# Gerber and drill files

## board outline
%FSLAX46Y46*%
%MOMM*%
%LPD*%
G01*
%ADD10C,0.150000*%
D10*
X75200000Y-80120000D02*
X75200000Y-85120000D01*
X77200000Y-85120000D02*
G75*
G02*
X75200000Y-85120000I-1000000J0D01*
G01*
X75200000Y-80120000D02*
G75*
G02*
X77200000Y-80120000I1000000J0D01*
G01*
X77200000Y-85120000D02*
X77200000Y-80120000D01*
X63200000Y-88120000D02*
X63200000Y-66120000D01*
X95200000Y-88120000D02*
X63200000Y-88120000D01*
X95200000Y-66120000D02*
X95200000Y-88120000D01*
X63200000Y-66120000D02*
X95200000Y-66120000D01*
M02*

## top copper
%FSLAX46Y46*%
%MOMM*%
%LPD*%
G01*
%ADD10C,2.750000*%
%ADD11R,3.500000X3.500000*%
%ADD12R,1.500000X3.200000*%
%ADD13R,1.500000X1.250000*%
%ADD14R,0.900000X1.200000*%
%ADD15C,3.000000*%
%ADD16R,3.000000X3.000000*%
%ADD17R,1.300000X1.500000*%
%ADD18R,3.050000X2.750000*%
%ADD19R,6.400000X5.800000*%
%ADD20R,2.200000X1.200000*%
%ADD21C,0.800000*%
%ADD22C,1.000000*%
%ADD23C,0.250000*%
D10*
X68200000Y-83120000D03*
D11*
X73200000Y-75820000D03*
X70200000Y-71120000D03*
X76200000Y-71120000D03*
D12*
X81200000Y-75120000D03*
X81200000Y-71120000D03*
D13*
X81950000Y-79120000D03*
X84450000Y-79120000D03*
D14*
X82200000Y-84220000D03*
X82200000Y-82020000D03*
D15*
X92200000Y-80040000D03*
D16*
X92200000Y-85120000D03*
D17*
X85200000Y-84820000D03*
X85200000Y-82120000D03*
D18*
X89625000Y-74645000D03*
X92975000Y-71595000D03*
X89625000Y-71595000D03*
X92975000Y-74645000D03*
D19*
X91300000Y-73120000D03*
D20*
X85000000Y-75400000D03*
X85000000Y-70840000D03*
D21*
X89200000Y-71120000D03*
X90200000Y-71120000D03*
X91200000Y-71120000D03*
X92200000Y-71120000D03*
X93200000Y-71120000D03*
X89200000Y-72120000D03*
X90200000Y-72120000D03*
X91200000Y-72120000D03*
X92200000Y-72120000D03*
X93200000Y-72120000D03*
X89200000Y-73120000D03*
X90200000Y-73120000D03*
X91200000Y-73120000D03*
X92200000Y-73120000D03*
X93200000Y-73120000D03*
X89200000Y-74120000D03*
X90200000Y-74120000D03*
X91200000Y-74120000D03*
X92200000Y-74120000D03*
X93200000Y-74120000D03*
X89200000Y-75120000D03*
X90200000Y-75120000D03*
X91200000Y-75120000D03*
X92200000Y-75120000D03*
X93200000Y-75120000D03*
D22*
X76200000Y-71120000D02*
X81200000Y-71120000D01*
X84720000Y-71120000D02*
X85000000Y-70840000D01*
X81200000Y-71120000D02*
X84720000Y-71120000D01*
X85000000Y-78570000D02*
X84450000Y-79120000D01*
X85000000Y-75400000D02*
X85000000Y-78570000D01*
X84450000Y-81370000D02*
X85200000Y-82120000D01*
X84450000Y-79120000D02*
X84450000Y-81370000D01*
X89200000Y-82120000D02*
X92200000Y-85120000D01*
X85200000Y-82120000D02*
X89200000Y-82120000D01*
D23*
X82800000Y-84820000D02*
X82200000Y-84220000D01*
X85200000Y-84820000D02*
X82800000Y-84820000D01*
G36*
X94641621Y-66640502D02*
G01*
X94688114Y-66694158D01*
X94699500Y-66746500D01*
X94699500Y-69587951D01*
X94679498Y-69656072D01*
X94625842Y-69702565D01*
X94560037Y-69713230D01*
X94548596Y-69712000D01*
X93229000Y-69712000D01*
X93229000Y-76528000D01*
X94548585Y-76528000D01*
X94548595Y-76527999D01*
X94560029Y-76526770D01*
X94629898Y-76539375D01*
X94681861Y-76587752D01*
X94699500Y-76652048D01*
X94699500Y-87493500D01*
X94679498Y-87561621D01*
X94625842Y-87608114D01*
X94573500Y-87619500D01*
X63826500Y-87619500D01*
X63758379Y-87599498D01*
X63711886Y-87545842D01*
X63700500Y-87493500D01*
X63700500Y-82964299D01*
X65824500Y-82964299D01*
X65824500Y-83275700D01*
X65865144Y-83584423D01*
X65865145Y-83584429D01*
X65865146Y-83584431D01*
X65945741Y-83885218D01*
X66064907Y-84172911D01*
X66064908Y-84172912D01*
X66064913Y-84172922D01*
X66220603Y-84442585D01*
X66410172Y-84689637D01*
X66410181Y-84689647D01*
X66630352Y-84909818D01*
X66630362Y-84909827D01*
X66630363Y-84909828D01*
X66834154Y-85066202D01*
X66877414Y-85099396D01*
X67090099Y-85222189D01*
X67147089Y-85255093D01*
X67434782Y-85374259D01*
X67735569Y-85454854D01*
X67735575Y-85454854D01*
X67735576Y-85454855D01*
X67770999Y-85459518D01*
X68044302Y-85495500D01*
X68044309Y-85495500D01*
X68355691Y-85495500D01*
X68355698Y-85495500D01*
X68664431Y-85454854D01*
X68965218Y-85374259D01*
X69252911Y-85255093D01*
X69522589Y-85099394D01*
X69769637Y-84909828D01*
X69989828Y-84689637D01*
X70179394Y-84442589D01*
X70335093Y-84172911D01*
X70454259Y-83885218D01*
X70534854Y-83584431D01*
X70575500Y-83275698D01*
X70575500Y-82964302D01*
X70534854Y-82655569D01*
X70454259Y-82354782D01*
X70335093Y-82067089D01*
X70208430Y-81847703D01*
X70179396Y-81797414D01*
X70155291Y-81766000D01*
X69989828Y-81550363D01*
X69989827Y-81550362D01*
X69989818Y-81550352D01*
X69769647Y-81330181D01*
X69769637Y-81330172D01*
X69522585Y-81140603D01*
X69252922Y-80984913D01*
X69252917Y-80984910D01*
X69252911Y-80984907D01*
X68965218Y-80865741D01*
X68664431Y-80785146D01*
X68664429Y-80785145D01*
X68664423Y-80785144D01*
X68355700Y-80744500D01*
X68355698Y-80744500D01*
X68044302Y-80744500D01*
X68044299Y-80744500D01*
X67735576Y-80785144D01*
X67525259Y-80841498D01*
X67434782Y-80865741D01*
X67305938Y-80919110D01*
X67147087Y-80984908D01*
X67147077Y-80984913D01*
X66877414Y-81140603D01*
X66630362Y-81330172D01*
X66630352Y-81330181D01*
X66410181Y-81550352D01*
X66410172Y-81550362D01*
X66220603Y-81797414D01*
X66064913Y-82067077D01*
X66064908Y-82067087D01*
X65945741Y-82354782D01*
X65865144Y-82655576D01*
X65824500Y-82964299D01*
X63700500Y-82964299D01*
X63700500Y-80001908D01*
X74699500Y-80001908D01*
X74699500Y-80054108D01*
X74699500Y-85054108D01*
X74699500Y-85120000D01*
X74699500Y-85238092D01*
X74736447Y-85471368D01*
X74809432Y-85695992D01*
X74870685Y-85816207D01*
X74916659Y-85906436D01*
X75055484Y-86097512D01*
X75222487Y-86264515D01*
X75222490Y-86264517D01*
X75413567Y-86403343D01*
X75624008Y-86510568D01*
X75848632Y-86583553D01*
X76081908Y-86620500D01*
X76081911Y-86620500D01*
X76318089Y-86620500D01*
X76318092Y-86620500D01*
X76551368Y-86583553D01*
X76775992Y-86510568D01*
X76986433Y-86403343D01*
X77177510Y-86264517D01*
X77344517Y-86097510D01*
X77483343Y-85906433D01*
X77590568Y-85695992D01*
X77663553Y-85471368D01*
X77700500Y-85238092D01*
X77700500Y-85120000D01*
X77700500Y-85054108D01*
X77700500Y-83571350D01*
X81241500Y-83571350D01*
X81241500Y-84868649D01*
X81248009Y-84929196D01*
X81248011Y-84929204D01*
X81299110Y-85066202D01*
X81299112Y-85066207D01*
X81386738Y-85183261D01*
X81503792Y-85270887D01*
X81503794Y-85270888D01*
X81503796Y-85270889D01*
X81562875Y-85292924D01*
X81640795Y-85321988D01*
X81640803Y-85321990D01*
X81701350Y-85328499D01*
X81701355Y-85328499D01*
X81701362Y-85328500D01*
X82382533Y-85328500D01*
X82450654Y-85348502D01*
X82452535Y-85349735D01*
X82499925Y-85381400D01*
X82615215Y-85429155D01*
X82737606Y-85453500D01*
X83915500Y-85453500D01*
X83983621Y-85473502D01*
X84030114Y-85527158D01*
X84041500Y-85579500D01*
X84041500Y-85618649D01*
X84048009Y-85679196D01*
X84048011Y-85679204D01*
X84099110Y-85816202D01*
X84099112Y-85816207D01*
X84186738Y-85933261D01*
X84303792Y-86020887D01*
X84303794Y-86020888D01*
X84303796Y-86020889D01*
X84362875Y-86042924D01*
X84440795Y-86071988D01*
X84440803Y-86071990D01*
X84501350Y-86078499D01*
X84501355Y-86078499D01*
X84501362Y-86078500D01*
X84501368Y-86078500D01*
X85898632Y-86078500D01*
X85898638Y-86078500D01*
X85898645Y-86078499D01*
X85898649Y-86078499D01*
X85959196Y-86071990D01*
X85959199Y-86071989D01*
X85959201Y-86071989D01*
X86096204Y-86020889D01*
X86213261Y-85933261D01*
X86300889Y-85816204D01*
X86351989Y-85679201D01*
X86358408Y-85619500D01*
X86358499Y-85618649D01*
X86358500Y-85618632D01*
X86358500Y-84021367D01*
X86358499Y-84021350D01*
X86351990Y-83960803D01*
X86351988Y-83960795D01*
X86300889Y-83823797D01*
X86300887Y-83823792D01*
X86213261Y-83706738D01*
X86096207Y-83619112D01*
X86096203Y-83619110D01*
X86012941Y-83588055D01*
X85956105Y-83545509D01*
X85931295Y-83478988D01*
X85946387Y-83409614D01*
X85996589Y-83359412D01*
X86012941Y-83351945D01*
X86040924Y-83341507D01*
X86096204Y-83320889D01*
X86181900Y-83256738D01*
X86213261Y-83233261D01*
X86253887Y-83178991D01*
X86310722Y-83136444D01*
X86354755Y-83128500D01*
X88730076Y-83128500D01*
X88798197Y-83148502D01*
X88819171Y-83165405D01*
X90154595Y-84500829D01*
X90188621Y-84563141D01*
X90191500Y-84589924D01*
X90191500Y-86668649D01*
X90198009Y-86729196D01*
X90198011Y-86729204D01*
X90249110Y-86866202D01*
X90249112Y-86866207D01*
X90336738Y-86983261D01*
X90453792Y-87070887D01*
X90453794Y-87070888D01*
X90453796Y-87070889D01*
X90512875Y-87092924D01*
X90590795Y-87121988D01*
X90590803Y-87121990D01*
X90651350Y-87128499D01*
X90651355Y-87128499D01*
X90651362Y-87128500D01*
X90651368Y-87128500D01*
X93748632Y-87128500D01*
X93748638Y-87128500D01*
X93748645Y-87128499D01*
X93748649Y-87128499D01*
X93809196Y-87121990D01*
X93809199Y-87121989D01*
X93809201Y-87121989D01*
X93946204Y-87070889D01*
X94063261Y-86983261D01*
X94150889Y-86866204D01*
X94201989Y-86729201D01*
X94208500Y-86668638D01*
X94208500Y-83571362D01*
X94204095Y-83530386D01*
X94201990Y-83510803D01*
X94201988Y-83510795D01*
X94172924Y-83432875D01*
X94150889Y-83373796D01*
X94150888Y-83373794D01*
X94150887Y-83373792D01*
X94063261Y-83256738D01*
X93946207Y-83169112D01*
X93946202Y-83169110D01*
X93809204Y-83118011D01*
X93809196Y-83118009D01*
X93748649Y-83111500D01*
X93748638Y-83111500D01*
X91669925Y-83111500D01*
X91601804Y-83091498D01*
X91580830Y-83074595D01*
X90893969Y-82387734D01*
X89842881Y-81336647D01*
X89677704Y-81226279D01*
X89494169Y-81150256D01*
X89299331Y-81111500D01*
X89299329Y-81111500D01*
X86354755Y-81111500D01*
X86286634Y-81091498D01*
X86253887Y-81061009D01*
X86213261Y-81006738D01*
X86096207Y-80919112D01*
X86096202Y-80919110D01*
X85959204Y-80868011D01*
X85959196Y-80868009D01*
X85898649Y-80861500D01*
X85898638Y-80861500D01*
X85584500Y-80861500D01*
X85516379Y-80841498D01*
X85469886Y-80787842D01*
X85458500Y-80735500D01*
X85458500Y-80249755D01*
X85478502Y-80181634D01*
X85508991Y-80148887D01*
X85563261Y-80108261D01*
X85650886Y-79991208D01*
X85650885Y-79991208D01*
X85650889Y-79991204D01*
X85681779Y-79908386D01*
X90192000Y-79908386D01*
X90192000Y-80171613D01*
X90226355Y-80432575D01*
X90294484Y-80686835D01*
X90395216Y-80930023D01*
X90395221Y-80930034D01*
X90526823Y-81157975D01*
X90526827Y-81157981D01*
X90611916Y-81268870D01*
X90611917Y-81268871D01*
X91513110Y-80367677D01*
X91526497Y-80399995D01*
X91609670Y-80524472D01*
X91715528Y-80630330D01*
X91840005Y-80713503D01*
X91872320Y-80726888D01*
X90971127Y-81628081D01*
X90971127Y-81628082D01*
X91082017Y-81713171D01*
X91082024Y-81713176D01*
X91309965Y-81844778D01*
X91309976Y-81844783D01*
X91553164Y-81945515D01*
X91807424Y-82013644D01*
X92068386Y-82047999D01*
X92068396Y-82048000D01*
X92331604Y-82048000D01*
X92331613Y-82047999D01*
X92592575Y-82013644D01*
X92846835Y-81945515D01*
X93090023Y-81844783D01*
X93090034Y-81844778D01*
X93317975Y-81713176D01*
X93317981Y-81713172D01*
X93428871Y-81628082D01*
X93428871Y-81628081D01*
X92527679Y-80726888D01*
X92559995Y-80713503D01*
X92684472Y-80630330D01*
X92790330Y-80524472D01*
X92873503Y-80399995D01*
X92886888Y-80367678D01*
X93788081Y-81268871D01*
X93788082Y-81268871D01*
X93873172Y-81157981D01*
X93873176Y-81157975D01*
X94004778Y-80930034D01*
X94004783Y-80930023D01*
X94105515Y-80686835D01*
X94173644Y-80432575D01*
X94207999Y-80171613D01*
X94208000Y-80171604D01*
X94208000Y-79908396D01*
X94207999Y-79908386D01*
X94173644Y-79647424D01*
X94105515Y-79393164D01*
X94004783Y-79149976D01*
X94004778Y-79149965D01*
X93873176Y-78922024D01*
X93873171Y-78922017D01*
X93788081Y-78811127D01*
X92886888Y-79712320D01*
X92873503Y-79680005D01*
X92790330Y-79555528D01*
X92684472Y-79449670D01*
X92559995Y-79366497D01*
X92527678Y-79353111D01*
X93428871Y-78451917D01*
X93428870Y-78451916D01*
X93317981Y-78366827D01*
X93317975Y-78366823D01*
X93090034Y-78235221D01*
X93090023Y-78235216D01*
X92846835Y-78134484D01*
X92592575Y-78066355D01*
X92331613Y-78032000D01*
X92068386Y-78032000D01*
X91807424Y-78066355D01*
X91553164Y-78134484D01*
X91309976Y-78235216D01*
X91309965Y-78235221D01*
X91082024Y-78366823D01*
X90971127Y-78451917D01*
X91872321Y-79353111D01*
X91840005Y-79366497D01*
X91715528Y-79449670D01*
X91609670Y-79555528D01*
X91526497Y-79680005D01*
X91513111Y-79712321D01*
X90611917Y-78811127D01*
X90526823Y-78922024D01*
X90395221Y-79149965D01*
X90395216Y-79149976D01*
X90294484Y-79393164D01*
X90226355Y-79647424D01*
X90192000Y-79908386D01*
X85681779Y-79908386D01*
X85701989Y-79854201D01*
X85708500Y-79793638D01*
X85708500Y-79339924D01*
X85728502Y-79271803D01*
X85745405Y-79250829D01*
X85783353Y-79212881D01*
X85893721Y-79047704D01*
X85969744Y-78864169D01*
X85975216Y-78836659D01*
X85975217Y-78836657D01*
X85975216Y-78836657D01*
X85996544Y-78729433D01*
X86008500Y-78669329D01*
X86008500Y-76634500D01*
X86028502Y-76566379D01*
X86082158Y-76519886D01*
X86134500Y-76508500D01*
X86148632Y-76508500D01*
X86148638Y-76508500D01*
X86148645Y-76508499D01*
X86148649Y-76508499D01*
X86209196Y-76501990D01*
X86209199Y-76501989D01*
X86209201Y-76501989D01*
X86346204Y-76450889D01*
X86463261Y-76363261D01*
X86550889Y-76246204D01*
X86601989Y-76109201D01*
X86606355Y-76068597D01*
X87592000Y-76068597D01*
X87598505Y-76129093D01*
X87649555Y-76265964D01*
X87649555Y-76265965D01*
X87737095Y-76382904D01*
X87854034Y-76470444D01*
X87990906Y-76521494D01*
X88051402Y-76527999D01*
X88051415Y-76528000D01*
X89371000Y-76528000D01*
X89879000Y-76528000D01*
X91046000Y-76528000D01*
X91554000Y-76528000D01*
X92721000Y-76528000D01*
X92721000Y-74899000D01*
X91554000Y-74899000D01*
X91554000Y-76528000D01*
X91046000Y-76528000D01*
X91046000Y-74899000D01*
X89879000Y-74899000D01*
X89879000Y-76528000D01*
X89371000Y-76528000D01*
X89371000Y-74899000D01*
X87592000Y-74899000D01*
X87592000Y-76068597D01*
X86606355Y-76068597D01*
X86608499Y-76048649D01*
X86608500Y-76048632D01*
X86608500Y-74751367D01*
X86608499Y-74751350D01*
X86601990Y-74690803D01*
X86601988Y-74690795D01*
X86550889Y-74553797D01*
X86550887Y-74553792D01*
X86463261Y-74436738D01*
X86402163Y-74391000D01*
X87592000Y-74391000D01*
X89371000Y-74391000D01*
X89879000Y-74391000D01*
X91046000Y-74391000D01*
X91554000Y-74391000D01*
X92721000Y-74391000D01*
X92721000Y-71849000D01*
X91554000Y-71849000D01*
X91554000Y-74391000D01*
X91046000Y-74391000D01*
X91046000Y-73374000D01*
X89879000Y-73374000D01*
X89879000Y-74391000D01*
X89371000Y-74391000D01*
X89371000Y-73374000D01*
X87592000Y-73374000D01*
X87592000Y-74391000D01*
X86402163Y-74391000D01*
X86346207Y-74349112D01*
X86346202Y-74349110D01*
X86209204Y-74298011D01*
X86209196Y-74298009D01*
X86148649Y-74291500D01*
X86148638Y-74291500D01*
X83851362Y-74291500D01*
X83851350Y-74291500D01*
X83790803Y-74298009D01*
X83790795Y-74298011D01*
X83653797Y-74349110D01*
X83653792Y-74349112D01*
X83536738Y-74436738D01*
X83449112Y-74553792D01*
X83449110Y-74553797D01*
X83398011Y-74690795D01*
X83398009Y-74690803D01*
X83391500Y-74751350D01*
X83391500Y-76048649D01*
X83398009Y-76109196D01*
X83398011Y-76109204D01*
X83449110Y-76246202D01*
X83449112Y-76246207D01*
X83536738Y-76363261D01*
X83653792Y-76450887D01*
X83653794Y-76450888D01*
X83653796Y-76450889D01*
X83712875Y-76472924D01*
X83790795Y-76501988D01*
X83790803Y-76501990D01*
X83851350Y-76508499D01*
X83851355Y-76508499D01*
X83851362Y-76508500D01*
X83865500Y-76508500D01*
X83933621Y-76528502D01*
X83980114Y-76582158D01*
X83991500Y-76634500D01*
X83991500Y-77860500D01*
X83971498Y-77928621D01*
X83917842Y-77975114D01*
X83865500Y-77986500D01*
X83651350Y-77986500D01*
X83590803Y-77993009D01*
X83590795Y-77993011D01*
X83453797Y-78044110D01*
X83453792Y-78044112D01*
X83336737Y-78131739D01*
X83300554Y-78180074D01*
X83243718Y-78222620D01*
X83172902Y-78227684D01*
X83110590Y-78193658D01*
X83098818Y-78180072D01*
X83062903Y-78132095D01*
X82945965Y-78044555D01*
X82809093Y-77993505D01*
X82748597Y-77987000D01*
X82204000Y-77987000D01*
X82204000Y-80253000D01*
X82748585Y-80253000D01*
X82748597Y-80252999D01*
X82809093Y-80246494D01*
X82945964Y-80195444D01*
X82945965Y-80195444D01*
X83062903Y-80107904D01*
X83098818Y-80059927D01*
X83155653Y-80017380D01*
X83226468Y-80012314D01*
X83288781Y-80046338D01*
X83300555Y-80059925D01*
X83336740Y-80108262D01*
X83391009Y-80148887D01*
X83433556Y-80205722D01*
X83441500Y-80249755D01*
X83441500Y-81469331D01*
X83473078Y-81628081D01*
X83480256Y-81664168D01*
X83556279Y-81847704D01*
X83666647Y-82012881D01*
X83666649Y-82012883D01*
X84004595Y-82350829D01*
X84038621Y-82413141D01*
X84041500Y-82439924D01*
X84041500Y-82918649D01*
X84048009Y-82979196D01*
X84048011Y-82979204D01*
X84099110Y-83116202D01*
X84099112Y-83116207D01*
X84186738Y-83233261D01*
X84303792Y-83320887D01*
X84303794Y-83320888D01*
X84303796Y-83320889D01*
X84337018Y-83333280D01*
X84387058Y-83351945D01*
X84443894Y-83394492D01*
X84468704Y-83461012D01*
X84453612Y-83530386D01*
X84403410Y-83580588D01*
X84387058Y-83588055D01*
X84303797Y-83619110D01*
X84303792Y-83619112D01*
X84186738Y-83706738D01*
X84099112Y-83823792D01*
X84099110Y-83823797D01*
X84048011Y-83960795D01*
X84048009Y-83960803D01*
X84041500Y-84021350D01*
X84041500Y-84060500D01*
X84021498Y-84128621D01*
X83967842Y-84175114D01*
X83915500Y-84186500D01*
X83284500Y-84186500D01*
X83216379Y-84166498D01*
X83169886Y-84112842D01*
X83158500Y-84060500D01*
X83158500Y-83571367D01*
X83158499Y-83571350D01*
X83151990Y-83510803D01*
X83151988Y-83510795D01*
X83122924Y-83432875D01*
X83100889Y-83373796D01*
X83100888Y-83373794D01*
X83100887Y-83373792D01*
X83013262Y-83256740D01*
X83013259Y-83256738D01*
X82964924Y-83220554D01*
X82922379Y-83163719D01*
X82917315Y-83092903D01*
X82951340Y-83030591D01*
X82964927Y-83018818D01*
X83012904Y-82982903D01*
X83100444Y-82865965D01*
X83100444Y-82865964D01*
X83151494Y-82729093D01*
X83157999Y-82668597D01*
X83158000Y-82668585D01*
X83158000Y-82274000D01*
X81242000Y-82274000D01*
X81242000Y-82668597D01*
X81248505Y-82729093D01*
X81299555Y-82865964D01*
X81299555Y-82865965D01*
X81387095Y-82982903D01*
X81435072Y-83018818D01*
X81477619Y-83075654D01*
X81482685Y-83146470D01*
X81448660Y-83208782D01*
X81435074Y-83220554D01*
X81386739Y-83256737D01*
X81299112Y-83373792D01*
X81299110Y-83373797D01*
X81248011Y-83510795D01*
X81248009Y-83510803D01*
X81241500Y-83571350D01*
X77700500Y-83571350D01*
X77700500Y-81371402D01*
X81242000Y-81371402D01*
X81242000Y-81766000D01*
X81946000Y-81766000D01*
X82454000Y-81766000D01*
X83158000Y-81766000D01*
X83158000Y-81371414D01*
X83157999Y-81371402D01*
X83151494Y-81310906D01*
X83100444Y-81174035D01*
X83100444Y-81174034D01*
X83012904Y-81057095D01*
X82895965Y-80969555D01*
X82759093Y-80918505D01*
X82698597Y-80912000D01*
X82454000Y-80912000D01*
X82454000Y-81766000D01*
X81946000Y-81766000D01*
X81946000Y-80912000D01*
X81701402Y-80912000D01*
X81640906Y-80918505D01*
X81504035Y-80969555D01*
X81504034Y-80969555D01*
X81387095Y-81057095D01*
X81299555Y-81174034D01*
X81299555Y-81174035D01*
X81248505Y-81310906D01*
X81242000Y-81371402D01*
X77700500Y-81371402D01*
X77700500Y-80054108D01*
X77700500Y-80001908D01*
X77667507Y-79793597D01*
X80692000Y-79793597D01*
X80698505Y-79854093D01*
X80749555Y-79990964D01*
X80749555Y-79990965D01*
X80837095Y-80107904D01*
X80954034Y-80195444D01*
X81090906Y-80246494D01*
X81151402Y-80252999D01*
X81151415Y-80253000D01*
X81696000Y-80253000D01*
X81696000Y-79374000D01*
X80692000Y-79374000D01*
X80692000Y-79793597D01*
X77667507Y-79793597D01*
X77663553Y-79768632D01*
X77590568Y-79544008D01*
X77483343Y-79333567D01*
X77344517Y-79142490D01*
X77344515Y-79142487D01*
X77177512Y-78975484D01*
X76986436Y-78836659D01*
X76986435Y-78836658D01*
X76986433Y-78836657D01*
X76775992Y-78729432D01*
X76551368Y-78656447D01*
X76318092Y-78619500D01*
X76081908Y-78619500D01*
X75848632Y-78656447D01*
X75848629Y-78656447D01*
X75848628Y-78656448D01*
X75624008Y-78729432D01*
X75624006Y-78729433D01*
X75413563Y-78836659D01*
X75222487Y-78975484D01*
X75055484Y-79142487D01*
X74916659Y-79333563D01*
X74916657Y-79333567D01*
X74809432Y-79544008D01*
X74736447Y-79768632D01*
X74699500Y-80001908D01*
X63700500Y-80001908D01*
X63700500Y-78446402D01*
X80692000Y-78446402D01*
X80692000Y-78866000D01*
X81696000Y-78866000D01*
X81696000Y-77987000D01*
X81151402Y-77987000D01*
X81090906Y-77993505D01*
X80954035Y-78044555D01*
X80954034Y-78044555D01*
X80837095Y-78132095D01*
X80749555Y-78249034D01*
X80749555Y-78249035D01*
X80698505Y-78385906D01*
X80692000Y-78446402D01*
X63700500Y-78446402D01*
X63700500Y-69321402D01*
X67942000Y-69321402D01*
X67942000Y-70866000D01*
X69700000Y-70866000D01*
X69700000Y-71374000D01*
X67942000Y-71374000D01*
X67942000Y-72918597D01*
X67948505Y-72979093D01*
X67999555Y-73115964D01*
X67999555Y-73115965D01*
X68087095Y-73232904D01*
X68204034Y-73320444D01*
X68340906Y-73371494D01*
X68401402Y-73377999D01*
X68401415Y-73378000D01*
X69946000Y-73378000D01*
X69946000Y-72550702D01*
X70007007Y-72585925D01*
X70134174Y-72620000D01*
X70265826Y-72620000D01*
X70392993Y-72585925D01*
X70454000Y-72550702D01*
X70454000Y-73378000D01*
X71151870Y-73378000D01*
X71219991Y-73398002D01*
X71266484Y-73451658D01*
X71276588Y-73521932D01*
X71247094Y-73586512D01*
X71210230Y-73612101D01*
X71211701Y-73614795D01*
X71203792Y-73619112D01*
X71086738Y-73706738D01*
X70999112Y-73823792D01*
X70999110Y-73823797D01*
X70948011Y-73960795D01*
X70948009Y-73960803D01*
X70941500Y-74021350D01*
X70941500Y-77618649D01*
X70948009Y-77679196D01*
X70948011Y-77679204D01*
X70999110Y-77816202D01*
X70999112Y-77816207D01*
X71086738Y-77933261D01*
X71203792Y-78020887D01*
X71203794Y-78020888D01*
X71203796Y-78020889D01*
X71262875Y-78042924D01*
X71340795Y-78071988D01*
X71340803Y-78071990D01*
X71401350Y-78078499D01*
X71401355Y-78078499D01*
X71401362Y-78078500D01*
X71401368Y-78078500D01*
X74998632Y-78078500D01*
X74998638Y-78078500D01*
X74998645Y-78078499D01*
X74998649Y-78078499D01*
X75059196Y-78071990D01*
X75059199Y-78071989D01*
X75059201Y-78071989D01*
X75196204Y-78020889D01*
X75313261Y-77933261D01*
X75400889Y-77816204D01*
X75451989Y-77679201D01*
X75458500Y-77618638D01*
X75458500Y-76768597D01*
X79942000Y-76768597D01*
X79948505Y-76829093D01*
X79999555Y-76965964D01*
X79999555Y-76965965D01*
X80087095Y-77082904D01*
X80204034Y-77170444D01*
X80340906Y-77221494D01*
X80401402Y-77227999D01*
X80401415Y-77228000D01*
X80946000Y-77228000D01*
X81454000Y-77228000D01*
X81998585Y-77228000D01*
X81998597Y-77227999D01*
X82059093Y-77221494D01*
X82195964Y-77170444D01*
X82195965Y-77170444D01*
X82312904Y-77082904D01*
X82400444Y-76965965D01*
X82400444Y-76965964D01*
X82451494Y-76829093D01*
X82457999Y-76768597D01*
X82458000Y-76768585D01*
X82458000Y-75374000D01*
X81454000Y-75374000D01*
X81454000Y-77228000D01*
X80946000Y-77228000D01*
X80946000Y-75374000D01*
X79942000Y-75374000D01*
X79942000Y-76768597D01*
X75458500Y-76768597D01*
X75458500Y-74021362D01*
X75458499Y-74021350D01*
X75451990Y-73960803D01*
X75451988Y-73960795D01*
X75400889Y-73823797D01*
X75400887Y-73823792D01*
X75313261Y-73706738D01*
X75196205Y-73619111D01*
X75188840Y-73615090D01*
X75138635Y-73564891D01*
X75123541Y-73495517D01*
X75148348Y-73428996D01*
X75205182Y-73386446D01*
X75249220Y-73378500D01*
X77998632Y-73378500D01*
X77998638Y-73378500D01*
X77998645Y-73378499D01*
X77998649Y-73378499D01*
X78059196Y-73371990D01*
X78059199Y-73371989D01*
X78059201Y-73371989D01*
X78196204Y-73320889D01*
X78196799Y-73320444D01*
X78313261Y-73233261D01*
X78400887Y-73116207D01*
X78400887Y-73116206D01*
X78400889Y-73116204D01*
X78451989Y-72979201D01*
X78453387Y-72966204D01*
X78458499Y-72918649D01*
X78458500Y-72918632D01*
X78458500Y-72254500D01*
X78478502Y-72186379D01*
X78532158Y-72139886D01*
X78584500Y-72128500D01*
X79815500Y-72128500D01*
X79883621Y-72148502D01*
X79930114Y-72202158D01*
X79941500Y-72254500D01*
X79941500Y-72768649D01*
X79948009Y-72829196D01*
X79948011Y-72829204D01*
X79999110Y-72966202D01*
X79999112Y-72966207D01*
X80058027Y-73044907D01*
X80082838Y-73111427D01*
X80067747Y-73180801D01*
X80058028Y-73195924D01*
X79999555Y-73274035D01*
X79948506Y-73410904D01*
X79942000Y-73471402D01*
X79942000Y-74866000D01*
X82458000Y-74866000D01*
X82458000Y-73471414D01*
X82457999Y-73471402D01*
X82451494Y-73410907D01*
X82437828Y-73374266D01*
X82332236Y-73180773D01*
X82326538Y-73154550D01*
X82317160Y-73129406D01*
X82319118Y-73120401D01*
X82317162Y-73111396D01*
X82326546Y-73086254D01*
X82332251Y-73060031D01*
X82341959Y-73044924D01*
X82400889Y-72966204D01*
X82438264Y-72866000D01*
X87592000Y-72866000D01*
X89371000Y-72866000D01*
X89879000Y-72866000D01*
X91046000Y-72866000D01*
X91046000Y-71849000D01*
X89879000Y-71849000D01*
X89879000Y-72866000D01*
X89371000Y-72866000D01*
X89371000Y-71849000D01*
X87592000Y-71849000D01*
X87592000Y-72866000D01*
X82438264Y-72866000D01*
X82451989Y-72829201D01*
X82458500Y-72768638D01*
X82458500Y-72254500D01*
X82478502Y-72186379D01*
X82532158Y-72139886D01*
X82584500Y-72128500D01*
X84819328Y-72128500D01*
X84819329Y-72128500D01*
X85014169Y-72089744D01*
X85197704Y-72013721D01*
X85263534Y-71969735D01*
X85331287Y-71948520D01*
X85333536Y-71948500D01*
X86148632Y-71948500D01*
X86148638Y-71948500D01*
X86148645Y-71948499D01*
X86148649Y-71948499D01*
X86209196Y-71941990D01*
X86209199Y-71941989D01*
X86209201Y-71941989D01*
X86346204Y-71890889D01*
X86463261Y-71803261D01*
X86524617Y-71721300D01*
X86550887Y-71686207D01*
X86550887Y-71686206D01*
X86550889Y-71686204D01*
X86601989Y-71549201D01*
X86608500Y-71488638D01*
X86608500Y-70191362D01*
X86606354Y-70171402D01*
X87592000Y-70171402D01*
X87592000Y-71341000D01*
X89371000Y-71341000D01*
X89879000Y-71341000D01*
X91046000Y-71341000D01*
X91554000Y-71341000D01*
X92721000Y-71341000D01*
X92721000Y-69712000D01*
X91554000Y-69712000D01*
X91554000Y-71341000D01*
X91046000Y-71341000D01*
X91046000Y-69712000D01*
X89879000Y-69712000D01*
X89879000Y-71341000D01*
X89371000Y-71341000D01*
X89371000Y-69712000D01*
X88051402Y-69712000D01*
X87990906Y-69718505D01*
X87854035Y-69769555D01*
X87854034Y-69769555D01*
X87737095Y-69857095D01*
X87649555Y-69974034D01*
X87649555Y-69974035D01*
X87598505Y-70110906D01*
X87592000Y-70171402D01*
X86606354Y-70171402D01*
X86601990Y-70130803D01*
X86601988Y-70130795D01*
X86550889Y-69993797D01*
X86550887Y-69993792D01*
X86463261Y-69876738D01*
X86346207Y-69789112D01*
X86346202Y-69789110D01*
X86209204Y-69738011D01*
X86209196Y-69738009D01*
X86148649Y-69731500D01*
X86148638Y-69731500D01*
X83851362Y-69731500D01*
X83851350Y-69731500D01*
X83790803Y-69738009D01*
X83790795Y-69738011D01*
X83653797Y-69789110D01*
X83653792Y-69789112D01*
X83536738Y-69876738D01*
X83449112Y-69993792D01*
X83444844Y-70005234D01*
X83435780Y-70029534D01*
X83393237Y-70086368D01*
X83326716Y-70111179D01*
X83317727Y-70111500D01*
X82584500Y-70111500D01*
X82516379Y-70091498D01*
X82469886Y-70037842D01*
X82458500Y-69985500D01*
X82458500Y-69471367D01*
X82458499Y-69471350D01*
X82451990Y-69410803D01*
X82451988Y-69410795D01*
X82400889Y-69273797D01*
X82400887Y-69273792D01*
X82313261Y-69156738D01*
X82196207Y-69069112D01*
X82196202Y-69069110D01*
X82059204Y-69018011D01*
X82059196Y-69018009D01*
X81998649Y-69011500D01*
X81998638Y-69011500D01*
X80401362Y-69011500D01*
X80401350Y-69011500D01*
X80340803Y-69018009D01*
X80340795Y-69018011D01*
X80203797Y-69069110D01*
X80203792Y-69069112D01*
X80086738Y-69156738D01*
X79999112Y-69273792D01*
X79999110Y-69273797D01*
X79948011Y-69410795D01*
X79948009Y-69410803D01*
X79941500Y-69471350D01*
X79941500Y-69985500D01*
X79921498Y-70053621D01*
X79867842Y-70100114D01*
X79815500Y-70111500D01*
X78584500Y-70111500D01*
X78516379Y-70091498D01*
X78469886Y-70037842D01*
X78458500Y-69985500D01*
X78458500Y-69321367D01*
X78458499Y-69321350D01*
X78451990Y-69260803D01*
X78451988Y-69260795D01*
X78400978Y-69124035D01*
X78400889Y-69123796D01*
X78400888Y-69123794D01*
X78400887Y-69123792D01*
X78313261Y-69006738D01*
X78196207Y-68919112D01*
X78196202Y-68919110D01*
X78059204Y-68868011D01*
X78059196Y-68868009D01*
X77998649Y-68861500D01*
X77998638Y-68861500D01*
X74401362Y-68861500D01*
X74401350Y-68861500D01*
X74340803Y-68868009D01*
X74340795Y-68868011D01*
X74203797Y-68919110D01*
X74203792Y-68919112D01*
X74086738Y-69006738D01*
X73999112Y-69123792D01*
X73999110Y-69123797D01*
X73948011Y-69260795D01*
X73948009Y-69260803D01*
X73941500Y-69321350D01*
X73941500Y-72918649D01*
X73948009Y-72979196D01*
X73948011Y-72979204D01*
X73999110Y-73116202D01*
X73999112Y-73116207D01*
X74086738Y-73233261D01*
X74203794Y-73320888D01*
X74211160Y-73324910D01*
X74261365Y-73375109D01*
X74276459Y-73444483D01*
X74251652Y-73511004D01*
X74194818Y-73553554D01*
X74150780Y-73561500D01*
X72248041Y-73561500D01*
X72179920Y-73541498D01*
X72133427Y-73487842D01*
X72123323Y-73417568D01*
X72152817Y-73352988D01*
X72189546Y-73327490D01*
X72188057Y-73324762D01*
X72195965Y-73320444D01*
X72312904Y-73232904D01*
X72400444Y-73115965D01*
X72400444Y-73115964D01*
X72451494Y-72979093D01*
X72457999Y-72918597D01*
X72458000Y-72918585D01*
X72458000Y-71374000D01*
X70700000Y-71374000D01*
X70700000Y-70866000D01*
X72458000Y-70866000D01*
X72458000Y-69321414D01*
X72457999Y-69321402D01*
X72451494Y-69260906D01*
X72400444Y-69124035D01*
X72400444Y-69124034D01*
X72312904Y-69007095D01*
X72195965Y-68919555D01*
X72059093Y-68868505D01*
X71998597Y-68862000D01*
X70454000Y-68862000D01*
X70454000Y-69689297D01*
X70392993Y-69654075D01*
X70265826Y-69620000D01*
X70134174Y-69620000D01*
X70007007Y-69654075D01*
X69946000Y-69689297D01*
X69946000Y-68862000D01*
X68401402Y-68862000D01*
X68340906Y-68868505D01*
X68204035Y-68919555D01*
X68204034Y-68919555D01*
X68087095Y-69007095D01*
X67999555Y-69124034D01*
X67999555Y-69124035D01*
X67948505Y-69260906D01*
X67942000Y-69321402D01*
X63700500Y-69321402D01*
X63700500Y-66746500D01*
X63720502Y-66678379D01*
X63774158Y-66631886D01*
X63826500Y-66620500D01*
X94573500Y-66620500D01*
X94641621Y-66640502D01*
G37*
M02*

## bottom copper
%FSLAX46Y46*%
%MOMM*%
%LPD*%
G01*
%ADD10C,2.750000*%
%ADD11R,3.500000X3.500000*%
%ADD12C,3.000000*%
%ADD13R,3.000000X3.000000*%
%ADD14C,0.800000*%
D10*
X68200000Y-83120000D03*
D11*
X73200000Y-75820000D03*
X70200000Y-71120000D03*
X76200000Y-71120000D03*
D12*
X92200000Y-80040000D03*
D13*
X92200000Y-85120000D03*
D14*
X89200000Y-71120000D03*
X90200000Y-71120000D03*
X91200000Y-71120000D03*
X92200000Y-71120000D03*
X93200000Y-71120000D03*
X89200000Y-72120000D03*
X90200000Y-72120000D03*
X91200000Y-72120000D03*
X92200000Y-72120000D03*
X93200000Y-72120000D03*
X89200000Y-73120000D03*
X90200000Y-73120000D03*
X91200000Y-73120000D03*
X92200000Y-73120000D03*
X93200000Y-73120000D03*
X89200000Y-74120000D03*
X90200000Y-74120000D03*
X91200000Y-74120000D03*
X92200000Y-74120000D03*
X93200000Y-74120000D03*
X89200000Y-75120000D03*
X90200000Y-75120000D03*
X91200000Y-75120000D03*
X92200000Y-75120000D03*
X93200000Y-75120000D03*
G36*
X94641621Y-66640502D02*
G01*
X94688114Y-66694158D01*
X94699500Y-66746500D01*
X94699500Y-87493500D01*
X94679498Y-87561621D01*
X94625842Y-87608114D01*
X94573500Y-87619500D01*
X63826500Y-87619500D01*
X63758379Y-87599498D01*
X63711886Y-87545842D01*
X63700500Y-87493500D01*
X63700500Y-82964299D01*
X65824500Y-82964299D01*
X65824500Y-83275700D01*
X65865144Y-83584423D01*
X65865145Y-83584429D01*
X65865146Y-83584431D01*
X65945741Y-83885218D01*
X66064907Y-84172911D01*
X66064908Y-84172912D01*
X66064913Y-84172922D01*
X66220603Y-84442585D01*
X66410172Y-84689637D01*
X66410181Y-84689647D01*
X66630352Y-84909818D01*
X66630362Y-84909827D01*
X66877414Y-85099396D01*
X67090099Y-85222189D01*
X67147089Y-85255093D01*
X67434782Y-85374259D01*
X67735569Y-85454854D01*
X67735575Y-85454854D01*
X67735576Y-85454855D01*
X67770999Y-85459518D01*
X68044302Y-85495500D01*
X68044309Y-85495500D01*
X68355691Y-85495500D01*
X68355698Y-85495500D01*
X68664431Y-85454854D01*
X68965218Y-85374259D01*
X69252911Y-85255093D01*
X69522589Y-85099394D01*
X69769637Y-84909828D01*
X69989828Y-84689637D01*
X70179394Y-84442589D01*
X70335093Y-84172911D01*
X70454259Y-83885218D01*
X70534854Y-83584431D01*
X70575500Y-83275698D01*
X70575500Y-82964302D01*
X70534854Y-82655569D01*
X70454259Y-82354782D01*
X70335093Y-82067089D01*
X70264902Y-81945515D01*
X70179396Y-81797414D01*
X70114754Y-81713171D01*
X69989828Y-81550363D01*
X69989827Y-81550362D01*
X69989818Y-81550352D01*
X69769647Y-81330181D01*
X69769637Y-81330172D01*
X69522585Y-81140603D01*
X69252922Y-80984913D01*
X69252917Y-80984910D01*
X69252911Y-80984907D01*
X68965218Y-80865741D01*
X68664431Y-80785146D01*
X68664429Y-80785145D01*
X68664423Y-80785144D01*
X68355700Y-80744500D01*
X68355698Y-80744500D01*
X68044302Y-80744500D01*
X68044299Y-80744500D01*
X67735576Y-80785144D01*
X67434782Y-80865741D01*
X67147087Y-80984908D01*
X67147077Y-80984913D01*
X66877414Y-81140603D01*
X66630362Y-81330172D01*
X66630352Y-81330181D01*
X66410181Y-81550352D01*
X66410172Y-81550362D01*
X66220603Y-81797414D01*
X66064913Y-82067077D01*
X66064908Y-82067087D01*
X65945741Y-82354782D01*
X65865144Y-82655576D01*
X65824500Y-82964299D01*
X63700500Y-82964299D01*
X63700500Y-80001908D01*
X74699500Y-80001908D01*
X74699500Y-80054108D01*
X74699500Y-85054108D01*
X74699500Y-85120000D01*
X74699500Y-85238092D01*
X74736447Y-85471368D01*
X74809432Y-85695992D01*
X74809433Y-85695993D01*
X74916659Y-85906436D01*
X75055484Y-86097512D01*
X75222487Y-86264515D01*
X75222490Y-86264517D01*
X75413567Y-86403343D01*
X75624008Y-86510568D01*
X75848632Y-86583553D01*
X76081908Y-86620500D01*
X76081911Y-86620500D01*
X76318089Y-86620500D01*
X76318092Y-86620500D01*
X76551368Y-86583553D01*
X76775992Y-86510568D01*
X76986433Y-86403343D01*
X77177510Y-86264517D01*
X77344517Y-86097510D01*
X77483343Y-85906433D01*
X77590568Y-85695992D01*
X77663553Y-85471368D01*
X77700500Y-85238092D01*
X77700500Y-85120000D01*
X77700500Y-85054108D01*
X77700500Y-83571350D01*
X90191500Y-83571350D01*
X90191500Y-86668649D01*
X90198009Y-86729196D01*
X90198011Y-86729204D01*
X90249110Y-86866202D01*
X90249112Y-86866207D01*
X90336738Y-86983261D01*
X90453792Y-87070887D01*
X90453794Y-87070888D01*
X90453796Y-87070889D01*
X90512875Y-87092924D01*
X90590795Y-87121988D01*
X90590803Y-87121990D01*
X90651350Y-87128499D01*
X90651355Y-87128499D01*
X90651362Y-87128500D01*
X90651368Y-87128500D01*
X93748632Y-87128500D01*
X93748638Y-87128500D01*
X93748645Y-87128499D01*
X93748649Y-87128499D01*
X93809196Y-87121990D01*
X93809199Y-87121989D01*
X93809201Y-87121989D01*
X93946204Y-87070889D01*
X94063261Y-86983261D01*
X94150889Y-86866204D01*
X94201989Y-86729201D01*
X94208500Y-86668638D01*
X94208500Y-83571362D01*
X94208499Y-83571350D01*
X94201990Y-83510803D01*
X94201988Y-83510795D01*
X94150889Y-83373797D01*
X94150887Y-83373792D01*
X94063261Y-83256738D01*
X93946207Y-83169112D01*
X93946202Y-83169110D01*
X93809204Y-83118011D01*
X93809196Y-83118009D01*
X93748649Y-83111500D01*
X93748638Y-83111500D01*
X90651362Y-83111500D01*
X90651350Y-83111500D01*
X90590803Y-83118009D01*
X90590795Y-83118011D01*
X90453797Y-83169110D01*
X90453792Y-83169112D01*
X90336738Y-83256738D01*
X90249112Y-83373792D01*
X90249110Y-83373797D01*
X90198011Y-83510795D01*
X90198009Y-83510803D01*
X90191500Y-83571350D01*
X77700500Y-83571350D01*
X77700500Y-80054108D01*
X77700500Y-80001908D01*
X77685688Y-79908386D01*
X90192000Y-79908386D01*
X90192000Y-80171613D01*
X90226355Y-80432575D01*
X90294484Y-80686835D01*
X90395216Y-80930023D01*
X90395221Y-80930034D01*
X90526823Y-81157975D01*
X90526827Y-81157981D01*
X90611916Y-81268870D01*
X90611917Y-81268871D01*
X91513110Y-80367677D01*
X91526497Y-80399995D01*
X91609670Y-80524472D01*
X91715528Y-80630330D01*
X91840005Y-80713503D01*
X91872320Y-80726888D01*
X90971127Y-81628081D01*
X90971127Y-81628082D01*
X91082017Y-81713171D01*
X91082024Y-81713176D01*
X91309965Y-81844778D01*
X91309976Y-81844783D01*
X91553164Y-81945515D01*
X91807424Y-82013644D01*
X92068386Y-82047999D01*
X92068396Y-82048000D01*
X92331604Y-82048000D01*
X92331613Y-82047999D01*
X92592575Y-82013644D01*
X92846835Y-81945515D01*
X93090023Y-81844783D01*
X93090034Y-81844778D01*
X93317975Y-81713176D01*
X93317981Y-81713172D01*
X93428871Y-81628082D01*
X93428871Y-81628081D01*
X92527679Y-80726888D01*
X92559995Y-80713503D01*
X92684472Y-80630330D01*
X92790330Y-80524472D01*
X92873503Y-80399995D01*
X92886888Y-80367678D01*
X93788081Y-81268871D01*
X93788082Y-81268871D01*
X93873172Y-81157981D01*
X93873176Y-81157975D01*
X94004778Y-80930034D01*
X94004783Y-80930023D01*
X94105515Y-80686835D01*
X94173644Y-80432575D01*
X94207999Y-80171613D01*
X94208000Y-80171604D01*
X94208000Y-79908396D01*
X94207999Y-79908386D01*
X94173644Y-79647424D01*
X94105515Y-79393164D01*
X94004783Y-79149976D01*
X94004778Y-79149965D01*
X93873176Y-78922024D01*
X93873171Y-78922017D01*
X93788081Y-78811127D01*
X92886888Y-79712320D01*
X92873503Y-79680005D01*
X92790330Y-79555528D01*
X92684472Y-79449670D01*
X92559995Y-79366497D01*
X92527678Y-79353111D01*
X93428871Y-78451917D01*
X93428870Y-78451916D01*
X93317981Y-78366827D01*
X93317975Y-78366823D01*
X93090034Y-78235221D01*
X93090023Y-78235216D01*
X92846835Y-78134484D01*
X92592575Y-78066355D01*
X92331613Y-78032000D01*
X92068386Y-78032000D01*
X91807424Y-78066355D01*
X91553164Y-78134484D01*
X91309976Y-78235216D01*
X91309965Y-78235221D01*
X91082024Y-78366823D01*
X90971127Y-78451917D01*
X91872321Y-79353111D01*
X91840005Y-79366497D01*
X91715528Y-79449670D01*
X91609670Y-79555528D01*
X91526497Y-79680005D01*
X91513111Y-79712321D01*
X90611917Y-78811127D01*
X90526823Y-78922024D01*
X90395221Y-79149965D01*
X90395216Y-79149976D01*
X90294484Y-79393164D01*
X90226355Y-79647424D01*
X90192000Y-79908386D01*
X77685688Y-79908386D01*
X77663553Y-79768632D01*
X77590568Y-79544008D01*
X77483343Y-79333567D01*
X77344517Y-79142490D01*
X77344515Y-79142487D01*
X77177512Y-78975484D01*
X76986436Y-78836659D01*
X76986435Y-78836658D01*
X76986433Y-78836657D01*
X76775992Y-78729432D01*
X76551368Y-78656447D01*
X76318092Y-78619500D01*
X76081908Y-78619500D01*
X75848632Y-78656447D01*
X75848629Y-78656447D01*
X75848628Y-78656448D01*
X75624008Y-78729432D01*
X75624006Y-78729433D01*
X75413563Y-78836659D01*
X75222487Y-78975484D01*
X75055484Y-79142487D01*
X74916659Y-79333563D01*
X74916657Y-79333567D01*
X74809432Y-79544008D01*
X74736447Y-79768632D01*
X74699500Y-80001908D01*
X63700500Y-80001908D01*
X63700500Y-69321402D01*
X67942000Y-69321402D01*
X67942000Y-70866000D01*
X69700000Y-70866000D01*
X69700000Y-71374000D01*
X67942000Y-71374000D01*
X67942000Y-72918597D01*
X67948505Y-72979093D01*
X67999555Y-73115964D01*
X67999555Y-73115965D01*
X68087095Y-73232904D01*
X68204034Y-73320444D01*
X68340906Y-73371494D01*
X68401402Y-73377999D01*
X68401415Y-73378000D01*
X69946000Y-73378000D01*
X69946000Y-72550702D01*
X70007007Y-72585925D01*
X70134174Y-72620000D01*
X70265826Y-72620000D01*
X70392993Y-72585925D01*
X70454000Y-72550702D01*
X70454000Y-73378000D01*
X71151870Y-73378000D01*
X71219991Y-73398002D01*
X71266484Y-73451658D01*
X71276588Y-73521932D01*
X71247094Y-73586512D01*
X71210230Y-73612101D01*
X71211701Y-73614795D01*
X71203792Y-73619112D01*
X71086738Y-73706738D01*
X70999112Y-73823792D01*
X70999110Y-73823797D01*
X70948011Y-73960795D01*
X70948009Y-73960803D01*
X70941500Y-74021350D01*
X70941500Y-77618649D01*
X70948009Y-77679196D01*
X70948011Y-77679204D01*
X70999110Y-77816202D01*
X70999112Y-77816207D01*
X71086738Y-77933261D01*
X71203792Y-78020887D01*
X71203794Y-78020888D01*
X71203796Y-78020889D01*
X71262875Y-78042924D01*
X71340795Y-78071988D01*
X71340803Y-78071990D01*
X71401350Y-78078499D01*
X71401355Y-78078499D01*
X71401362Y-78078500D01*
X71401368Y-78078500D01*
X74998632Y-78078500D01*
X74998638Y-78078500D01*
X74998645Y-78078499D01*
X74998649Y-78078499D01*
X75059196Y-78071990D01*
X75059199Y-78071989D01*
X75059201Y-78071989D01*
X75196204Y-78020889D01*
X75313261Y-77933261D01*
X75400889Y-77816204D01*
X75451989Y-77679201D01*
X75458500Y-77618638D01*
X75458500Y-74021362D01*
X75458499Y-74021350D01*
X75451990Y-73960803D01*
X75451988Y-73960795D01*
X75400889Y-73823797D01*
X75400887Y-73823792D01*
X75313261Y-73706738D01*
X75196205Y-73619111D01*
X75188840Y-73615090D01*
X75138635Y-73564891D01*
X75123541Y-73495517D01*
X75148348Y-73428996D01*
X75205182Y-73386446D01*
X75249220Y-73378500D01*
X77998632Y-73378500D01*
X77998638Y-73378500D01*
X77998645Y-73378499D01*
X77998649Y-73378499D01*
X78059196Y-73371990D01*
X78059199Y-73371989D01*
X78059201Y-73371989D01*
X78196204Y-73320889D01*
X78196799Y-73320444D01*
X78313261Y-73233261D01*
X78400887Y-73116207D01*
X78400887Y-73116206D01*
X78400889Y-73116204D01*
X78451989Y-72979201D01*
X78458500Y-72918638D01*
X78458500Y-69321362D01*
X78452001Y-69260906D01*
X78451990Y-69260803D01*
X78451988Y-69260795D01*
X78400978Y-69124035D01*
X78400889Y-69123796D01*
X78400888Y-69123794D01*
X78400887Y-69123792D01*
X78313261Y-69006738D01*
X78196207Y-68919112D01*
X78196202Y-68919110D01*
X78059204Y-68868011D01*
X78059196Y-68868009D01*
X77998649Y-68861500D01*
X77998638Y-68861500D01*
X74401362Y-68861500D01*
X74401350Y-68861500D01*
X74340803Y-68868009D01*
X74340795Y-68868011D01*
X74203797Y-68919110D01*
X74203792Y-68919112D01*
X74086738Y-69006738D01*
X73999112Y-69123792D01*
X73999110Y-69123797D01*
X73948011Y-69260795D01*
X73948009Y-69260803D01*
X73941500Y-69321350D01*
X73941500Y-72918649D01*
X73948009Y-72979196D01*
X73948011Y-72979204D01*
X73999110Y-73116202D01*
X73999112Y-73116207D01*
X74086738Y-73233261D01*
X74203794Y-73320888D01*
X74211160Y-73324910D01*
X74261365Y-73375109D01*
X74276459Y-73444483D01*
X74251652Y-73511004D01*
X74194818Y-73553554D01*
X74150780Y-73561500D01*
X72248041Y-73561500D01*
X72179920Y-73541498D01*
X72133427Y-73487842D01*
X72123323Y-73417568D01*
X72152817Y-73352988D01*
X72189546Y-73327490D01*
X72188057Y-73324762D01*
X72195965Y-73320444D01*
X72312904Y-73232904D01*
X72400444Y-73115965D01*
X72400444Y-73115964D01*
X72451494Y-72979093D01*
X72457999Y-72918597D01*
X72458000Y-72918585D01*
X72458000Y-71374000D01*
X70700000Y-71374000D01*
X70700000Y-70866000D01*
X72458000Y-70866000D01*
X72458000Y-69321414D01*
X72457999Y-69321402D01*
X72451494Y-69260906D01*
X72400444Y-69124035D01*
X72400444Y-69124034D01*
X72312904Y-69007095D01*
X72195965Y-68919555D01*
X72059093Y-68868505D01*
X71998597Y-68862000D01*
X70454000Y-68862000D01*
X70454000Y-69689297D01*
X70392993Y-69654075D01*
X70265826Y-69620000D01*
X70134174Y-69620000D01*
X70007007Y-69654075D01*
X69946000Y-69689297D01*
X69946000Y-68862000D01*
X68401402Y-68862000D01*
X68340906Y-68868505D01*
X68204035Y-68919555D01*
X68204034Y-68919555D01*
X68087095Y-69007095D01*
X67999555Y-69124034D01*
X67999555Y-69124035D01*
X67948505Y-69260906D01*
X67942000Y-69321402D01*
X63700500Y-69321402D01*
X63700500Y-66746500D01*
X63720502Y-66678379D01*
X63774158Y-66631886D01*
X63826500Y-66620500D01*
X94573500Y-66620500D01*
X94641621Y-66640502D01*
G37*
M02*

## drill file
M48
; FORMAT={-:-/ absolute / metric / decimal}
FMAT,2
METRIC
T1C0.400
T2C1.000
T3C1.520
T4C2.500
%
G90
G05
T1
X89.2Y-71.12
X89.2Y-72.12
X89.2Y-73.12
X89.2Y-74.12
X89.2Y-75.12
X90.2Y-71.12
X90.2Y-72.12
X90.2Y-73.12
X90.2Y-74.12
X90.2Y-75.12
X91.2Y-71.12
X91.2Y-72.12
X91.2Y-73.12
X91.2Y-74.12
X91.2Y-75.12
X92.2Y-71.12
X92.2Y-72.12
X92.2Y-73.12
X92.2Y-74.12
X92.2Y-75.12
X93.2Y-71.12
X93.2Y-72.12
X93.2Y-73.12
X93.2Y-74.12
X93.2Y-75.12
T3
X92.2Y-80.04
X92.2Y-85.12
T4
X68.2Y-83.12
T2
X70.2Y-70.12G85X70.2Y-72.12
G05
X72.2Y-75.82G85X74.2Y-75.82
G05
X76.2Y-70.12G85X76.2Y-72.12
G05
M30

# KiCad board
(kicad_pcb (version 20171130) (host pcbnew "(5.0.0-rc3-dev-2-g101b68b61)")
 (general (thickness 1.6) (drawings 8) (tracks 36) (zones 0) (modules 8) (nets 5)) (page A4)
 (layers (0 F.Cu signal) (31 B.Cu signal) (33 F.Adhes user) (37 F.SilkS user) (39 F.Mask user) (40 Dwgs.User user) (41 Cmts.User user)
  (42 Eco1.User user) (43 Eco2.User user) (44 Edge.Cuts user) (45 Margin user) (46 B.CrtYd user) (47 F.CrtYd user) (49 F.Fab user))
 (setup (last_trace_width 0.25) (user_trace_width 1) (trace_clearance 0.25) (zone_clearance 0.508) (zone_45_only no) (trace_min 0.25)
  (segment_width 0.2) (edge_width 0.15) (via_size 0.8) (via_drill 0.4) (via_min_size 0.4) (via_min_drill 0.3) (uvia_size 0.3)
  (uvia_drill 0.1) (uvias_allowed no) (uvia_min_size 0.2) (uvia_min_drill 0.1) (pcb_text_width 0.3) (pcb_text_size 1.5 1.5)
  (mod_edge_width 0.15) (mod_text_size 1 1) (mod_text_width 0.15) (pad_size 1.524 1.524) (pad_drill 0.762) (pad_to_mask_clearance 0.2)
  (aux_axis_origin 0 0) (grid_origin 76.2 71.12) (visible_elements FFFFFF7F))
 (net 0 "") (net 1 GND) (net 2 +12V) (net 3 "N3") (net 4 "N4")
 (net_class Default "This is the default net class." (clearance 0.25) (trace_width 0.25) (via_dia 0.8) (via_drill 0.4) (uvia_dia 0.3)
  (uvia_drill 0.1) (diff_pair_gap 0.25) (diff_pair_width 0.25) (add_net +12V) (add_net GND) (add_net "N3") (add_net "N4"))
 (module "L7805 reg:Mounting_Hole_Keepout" (layer F.Cu) (at 68.2 83.12)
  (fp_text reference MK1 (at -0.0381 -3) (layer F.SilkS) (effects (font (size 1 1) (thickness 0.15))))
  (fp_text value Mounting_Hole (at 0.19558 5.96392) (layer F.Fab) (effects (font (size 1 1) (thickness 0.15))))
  (pad "" np_thru_hole circle (at 0 0) (size 2.75 2.75) (drill 2.5) (layers *.Cu *.Mask) (clearance 1)))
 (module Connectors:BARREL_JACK (layer F.Cu) (at 76.2 71.12)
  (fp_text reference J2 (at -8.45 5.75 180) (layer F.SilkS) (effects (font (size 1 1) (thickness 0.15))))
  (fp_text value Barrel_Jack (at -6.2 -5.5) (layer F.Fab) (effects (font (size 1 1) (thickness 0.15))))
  (pad 3 thru_hole rect (at -3 4.7) (size 3.5 3.5) (drill oval 3 1) (layers *.Cu *.Mask))
  (pad 2 thru_hole rect (at -6 0) (size 3.5 3.5) (drill oval 1 3) (layers *.Cu *.Mask) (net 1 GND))
  (pad 1 thru_hole rect (at 0 0) (size 3.5 3.5) (drill oval 1 3) (layers *.Cu *.Mask) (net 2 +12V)))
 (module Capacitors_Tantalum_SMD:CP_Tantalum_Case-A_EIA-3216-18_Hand (layer F.Cu) (at 81.2 73.12 270)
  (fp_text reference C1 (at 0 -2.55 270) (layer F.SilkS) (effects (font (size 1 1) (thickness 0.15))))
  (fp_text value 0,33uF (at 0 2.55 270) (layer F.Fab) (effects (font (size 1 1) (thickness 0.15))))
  (pad 2 smd rect (at 2 0 270) (size 3.2 1.5) (layers F.Cu F.Paste F.Mask) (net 1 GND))
  (pad 1 smd rect (at -2 0 270) (size 3.2 1.5) (layers F.Cu F.Paste F.Mask) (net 2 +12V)))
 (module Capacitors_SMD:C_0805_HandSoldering (layer F.Cu) (at 83.2 79.12 180)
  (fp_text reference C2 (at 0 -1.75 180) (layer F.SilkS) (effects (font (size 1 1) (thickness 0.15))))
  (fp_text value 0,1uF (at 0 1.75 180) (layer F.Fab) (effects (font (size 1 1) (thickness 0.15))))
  (pad 2 smd rect (at 1.25 0 180) (size 1.5 1.25) (layers F.Cu F.Paste F.Mask) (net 1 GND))
  (pad 1 smd rect (at -1.25 0 180) (size 1.5 1.25) (layers F.Cu F.Paste F.Mask) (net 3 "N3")))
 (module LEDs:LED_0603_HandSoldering (layer F.Cu) (at 82.2 83.12 270)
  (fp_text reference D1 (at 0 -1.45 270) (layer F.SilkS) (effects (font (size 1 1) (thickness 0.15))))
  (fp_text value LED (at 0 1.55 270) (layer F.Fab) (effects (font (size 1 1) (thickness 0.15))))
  (pad 2 smd rect (at 1.1 0 270) (size 1.2 0.9) (layers F.Cu F.Paste F.Mask) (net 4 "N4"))
  (pad 1 smd rect (at -1.1 0 270) (size 1.2 0.9) (layers F.Cu F.Paste F.Mask) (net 1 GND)))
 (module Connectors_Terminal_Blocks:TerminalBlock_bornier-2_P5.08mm (layer F.Cu) (at 92.2 85.12 90)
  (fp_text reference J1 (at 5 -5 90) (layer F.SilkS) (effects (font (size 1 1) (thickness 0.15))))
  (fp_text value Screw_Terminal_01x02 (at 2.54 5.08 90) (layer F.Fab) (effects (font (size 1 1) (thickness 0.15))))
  (pad 2 thru_hole circle (at 5.08 0 90) (size 3 3) (drill 1.52) (layers *.Cu *.Mask) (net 1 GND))
  (pad 1 thru_hole rect (at 0 0 90) (size 3 3) (drill 1.52) (layers *.Cu *.Mask) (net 3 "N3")))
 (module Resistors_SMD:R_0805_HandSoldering (layer F.Cu) (at 85.2 83.47 270)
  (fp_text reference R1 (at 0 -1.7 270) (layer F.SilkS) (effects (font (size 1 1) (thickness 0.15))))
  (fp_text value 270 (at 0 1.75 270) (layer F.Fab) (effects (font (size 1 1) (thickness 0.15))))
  (pad 2 smd rect (at 1.35 0 270) (size 1.5 1.3) (layers F.Cu F.Paste F.Mask) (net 4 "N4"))
  (pad 1 smd rect (at -1.35 0 270) (size 1.5 1.3) (layers F.Cu F.Paste F.Mask) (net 3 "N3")))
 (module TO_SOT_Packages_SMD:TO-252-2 (layer F.Cu) (at 89.2 73.12)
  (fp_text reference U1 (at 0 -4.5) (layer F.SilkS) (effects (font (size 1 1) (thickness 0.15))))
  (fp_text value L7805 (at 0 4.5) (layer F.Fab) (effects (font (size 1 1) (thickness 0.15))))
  (pad 2 smd rect (at 0.425 1.525) (size 3.05 2.75) (layers F.Cu F.Paste) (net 1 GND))
  (pad 2 smd rect (at 3.775 -1.525) (size 3.05 2.75) (layers F.Cu F.Paste) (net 1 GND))
  (pad 2 smd rect (at 0.425 -1.525) (size 3.05 2.75) (layers F.Cu F.Paste) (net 1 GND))
  (pad 2 smd rect (at 3.775 1.525) (size 3.05 2.75) (layers F.Cu F.Paste) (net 1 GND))
  (pad 2 smd rect (at 2.1 0) (size 6.4 5.8) (layers F.Cu F.Mask) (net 1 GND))
  (pad 3 smd rect (at -4.2 2.28) (size 2.2 1.2) (layers F.Cu F.Paste F.Mask) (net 3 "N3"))
  (pad 1 smd rect (at -4.2 -2.28) (size 2.2 1.2) (layers F.Cu F.Paste F.Mask) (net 2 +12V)))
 (gr_line (start 75.2 80.12) (end 75.2 85.12) (layer Edge.Cuts) (width 0.15))
 (gr_arc (start 76.2 85.12) (end 75.2 85.12) (angle -180) (layer Edge.Cuts) (width 0.15))
 (gr_arc (start 76.2 80.12) (end 77.2 80.12) (angle -180) (layer Edge.Cuts) (width 0.15))
 (gr_line (start 77.2 85.12) (end 77.2 80.12) (layer Edge.Cuts) (width 0.15))
 (gr_line (start 63.2 88.12) (end 63.2 66.12) (layer Edge.Cuts) (width 0.15))
 (gr_line (start 95.2 88.12) (end 63.2 88.12) (layer Edge.Cuts) (width 0.15))
 (gr_line (start 95.2 66.12) (end 95.2 88.12) (layer Edge.Cuts) (width 0.15))
 (gr_line (start 63.2 66.12) (end 95.2 66.12) (layer Edge.Cuts) (width 0.15))
 (via (at 89.2 71.12) (size 0.8) (drill 0.4) (layers F.Cu B.Cu) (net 1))
 (via (at 90.2 71.12) (size 0.8) (drill 0.4) (layers F.Cu B.Cu) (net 1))
 (via (at 91.2 71.12) (size 0.8) (drill 0.4) (layers F.Cu B.Cu) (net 1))
 (via (at 92.2 71.12) (size 0.8) (drill 0.4) (layers F.Cu B.Cu) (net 1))
 (via (at 93.2 71.12) (size 0.8) (drill 0.4) (layers F.Cu B.Cu) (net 1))
 (via (at 89.2 72.12) (size 0.8) (drill 0.4) (layers F.Cu B.Cu) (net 1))
 (via (at 90.2 72.12) (size 0.8) (drill 0.4) (layers F.Cu B.Cu) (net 1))
 (via (at 91.2 72.12) (size 0.8) (drill 0.4) (layers F.Cu B.Cu) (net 1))
 (via (at 92.2 72.12) (size 0.8) (drill 0.4) (layers F.Cu B.Cu) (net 1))
 (via (at 93.2 72.12) (size 0.8) (drill 0.4) (layers F.Cu B.Cu) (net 1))
 (via (at 89.2 73.12) (size 0.8) (drill 0.4) (layers F.Cu B.Cu) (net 1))
 (via (at 90.2 73.12) (size 0.8) (drill 0.4) (layers F.Cu B.Cu) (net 1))
 (via (at 91.2 73.12) (size 0.8) (drill 0.4) (layers F.Cu B.Cu) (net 1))
 (via (at 92.2 73.12) (size 0.8) (drill 0.4) (layers F.Cu B.Cu) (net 1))
 (via (at 93.2 73.12) (size 0.8) (drill 0.4) (layers F.Cu B.Cu) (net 1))
 (via (at 89.2 74.12) (size 0.8) (drill 0.4) (layers F.Cu B.Cu) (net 1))
 (via (at 90.2 74.12) (size 0.8) (drill 0.4) (layers F.Cu B.Cu) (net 1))
 (via (at 91.2 74.12) (size 0.8) (drill 0.4) (layers F.Cu B.Cu) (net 1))
 (via (at 92.2 74.12) (size 0.8) (drill 0.4) (layers F.Cu B.Cu) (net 1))
 (via (at 93.2 74.12) (size 0.8) (drill 0.4) (layers F.Cu B.Cu) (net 1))
 (via (at 89.2 75.12) (size 0.8) (drill 0.4) (layers F.Cu B.Cu) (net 1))
 (via (at 90.2 75.12) (size 0.8) (drill 0.4) (layers F.Cu B.Cu) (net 1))
 (via (at 91.2 75.12) (size 0.8) (drill 0.4) (layers F.Cu B.Cu) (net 1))
 (via (at 92.2 75.12) (size 0.8) (drill 0.4) (layers F.Cu B.Cu) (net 1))
 (via (at 93.2 75.12) (size 0.8) (drill 0.4) (layers F.Cu B.Cu) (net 1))
 (segment (start 76.2 71.12) (end 81.2 71.12) (width 1) (layer F.Cu) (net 2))
 (segment (start 84.72 71.12) (end 85 70.84) (width 1) (layer F.Cu) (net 2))
 (segment (start 81.2 71.12) (end 84.72 71.12) (width 1) (layer F.Cu) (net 2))
 (segment (start 85 78.57) (end 84.45 79.12) (width 1) (layer F.Cu) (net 3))
 (segment (start 85 75.4) (end 85 78.57) (width 1) (layer F.Cu) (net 3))
 (segment (start 84.45 81.37) (end 85.2 82.12) (width 1) (layer F.Cu) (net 3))
 (segment (start 84.45 79.12) (end 84.45 81.37) (width 1) (layer F.Cu) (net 3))
 (segment (start 89.2 82.12) (end 92.2 85.12) (width 1) (layer F.Cu) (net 3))
 (segment (start 85.2 82.12) (end 89.2 82.12) (width 1) (layer F.Cu) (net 3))
 (segment (start 82.8 84.82) (end 82.2 84.22) (width 0.25) (layer F.Cu) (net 4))
 (segment (start 85.2 84.82) (end 82.8 84.82) (width 0.25) (layer F.Cu) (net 4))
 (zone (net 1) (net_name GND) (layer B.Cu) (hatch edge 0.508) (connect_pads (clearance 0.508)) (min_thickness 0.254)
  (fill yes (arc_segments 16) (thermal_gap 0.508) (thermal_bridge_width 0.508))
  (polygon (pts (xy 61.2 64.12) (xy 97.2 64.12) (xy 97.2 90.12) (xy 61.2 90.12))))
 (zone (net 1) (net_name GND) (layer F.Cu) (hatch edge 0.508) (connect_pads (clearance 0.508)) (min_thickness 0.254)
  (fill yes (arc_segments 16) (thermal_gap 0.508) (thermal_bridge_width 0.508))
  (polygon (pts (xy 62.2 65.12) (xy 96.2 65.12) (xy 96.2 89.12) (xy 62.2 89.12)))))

